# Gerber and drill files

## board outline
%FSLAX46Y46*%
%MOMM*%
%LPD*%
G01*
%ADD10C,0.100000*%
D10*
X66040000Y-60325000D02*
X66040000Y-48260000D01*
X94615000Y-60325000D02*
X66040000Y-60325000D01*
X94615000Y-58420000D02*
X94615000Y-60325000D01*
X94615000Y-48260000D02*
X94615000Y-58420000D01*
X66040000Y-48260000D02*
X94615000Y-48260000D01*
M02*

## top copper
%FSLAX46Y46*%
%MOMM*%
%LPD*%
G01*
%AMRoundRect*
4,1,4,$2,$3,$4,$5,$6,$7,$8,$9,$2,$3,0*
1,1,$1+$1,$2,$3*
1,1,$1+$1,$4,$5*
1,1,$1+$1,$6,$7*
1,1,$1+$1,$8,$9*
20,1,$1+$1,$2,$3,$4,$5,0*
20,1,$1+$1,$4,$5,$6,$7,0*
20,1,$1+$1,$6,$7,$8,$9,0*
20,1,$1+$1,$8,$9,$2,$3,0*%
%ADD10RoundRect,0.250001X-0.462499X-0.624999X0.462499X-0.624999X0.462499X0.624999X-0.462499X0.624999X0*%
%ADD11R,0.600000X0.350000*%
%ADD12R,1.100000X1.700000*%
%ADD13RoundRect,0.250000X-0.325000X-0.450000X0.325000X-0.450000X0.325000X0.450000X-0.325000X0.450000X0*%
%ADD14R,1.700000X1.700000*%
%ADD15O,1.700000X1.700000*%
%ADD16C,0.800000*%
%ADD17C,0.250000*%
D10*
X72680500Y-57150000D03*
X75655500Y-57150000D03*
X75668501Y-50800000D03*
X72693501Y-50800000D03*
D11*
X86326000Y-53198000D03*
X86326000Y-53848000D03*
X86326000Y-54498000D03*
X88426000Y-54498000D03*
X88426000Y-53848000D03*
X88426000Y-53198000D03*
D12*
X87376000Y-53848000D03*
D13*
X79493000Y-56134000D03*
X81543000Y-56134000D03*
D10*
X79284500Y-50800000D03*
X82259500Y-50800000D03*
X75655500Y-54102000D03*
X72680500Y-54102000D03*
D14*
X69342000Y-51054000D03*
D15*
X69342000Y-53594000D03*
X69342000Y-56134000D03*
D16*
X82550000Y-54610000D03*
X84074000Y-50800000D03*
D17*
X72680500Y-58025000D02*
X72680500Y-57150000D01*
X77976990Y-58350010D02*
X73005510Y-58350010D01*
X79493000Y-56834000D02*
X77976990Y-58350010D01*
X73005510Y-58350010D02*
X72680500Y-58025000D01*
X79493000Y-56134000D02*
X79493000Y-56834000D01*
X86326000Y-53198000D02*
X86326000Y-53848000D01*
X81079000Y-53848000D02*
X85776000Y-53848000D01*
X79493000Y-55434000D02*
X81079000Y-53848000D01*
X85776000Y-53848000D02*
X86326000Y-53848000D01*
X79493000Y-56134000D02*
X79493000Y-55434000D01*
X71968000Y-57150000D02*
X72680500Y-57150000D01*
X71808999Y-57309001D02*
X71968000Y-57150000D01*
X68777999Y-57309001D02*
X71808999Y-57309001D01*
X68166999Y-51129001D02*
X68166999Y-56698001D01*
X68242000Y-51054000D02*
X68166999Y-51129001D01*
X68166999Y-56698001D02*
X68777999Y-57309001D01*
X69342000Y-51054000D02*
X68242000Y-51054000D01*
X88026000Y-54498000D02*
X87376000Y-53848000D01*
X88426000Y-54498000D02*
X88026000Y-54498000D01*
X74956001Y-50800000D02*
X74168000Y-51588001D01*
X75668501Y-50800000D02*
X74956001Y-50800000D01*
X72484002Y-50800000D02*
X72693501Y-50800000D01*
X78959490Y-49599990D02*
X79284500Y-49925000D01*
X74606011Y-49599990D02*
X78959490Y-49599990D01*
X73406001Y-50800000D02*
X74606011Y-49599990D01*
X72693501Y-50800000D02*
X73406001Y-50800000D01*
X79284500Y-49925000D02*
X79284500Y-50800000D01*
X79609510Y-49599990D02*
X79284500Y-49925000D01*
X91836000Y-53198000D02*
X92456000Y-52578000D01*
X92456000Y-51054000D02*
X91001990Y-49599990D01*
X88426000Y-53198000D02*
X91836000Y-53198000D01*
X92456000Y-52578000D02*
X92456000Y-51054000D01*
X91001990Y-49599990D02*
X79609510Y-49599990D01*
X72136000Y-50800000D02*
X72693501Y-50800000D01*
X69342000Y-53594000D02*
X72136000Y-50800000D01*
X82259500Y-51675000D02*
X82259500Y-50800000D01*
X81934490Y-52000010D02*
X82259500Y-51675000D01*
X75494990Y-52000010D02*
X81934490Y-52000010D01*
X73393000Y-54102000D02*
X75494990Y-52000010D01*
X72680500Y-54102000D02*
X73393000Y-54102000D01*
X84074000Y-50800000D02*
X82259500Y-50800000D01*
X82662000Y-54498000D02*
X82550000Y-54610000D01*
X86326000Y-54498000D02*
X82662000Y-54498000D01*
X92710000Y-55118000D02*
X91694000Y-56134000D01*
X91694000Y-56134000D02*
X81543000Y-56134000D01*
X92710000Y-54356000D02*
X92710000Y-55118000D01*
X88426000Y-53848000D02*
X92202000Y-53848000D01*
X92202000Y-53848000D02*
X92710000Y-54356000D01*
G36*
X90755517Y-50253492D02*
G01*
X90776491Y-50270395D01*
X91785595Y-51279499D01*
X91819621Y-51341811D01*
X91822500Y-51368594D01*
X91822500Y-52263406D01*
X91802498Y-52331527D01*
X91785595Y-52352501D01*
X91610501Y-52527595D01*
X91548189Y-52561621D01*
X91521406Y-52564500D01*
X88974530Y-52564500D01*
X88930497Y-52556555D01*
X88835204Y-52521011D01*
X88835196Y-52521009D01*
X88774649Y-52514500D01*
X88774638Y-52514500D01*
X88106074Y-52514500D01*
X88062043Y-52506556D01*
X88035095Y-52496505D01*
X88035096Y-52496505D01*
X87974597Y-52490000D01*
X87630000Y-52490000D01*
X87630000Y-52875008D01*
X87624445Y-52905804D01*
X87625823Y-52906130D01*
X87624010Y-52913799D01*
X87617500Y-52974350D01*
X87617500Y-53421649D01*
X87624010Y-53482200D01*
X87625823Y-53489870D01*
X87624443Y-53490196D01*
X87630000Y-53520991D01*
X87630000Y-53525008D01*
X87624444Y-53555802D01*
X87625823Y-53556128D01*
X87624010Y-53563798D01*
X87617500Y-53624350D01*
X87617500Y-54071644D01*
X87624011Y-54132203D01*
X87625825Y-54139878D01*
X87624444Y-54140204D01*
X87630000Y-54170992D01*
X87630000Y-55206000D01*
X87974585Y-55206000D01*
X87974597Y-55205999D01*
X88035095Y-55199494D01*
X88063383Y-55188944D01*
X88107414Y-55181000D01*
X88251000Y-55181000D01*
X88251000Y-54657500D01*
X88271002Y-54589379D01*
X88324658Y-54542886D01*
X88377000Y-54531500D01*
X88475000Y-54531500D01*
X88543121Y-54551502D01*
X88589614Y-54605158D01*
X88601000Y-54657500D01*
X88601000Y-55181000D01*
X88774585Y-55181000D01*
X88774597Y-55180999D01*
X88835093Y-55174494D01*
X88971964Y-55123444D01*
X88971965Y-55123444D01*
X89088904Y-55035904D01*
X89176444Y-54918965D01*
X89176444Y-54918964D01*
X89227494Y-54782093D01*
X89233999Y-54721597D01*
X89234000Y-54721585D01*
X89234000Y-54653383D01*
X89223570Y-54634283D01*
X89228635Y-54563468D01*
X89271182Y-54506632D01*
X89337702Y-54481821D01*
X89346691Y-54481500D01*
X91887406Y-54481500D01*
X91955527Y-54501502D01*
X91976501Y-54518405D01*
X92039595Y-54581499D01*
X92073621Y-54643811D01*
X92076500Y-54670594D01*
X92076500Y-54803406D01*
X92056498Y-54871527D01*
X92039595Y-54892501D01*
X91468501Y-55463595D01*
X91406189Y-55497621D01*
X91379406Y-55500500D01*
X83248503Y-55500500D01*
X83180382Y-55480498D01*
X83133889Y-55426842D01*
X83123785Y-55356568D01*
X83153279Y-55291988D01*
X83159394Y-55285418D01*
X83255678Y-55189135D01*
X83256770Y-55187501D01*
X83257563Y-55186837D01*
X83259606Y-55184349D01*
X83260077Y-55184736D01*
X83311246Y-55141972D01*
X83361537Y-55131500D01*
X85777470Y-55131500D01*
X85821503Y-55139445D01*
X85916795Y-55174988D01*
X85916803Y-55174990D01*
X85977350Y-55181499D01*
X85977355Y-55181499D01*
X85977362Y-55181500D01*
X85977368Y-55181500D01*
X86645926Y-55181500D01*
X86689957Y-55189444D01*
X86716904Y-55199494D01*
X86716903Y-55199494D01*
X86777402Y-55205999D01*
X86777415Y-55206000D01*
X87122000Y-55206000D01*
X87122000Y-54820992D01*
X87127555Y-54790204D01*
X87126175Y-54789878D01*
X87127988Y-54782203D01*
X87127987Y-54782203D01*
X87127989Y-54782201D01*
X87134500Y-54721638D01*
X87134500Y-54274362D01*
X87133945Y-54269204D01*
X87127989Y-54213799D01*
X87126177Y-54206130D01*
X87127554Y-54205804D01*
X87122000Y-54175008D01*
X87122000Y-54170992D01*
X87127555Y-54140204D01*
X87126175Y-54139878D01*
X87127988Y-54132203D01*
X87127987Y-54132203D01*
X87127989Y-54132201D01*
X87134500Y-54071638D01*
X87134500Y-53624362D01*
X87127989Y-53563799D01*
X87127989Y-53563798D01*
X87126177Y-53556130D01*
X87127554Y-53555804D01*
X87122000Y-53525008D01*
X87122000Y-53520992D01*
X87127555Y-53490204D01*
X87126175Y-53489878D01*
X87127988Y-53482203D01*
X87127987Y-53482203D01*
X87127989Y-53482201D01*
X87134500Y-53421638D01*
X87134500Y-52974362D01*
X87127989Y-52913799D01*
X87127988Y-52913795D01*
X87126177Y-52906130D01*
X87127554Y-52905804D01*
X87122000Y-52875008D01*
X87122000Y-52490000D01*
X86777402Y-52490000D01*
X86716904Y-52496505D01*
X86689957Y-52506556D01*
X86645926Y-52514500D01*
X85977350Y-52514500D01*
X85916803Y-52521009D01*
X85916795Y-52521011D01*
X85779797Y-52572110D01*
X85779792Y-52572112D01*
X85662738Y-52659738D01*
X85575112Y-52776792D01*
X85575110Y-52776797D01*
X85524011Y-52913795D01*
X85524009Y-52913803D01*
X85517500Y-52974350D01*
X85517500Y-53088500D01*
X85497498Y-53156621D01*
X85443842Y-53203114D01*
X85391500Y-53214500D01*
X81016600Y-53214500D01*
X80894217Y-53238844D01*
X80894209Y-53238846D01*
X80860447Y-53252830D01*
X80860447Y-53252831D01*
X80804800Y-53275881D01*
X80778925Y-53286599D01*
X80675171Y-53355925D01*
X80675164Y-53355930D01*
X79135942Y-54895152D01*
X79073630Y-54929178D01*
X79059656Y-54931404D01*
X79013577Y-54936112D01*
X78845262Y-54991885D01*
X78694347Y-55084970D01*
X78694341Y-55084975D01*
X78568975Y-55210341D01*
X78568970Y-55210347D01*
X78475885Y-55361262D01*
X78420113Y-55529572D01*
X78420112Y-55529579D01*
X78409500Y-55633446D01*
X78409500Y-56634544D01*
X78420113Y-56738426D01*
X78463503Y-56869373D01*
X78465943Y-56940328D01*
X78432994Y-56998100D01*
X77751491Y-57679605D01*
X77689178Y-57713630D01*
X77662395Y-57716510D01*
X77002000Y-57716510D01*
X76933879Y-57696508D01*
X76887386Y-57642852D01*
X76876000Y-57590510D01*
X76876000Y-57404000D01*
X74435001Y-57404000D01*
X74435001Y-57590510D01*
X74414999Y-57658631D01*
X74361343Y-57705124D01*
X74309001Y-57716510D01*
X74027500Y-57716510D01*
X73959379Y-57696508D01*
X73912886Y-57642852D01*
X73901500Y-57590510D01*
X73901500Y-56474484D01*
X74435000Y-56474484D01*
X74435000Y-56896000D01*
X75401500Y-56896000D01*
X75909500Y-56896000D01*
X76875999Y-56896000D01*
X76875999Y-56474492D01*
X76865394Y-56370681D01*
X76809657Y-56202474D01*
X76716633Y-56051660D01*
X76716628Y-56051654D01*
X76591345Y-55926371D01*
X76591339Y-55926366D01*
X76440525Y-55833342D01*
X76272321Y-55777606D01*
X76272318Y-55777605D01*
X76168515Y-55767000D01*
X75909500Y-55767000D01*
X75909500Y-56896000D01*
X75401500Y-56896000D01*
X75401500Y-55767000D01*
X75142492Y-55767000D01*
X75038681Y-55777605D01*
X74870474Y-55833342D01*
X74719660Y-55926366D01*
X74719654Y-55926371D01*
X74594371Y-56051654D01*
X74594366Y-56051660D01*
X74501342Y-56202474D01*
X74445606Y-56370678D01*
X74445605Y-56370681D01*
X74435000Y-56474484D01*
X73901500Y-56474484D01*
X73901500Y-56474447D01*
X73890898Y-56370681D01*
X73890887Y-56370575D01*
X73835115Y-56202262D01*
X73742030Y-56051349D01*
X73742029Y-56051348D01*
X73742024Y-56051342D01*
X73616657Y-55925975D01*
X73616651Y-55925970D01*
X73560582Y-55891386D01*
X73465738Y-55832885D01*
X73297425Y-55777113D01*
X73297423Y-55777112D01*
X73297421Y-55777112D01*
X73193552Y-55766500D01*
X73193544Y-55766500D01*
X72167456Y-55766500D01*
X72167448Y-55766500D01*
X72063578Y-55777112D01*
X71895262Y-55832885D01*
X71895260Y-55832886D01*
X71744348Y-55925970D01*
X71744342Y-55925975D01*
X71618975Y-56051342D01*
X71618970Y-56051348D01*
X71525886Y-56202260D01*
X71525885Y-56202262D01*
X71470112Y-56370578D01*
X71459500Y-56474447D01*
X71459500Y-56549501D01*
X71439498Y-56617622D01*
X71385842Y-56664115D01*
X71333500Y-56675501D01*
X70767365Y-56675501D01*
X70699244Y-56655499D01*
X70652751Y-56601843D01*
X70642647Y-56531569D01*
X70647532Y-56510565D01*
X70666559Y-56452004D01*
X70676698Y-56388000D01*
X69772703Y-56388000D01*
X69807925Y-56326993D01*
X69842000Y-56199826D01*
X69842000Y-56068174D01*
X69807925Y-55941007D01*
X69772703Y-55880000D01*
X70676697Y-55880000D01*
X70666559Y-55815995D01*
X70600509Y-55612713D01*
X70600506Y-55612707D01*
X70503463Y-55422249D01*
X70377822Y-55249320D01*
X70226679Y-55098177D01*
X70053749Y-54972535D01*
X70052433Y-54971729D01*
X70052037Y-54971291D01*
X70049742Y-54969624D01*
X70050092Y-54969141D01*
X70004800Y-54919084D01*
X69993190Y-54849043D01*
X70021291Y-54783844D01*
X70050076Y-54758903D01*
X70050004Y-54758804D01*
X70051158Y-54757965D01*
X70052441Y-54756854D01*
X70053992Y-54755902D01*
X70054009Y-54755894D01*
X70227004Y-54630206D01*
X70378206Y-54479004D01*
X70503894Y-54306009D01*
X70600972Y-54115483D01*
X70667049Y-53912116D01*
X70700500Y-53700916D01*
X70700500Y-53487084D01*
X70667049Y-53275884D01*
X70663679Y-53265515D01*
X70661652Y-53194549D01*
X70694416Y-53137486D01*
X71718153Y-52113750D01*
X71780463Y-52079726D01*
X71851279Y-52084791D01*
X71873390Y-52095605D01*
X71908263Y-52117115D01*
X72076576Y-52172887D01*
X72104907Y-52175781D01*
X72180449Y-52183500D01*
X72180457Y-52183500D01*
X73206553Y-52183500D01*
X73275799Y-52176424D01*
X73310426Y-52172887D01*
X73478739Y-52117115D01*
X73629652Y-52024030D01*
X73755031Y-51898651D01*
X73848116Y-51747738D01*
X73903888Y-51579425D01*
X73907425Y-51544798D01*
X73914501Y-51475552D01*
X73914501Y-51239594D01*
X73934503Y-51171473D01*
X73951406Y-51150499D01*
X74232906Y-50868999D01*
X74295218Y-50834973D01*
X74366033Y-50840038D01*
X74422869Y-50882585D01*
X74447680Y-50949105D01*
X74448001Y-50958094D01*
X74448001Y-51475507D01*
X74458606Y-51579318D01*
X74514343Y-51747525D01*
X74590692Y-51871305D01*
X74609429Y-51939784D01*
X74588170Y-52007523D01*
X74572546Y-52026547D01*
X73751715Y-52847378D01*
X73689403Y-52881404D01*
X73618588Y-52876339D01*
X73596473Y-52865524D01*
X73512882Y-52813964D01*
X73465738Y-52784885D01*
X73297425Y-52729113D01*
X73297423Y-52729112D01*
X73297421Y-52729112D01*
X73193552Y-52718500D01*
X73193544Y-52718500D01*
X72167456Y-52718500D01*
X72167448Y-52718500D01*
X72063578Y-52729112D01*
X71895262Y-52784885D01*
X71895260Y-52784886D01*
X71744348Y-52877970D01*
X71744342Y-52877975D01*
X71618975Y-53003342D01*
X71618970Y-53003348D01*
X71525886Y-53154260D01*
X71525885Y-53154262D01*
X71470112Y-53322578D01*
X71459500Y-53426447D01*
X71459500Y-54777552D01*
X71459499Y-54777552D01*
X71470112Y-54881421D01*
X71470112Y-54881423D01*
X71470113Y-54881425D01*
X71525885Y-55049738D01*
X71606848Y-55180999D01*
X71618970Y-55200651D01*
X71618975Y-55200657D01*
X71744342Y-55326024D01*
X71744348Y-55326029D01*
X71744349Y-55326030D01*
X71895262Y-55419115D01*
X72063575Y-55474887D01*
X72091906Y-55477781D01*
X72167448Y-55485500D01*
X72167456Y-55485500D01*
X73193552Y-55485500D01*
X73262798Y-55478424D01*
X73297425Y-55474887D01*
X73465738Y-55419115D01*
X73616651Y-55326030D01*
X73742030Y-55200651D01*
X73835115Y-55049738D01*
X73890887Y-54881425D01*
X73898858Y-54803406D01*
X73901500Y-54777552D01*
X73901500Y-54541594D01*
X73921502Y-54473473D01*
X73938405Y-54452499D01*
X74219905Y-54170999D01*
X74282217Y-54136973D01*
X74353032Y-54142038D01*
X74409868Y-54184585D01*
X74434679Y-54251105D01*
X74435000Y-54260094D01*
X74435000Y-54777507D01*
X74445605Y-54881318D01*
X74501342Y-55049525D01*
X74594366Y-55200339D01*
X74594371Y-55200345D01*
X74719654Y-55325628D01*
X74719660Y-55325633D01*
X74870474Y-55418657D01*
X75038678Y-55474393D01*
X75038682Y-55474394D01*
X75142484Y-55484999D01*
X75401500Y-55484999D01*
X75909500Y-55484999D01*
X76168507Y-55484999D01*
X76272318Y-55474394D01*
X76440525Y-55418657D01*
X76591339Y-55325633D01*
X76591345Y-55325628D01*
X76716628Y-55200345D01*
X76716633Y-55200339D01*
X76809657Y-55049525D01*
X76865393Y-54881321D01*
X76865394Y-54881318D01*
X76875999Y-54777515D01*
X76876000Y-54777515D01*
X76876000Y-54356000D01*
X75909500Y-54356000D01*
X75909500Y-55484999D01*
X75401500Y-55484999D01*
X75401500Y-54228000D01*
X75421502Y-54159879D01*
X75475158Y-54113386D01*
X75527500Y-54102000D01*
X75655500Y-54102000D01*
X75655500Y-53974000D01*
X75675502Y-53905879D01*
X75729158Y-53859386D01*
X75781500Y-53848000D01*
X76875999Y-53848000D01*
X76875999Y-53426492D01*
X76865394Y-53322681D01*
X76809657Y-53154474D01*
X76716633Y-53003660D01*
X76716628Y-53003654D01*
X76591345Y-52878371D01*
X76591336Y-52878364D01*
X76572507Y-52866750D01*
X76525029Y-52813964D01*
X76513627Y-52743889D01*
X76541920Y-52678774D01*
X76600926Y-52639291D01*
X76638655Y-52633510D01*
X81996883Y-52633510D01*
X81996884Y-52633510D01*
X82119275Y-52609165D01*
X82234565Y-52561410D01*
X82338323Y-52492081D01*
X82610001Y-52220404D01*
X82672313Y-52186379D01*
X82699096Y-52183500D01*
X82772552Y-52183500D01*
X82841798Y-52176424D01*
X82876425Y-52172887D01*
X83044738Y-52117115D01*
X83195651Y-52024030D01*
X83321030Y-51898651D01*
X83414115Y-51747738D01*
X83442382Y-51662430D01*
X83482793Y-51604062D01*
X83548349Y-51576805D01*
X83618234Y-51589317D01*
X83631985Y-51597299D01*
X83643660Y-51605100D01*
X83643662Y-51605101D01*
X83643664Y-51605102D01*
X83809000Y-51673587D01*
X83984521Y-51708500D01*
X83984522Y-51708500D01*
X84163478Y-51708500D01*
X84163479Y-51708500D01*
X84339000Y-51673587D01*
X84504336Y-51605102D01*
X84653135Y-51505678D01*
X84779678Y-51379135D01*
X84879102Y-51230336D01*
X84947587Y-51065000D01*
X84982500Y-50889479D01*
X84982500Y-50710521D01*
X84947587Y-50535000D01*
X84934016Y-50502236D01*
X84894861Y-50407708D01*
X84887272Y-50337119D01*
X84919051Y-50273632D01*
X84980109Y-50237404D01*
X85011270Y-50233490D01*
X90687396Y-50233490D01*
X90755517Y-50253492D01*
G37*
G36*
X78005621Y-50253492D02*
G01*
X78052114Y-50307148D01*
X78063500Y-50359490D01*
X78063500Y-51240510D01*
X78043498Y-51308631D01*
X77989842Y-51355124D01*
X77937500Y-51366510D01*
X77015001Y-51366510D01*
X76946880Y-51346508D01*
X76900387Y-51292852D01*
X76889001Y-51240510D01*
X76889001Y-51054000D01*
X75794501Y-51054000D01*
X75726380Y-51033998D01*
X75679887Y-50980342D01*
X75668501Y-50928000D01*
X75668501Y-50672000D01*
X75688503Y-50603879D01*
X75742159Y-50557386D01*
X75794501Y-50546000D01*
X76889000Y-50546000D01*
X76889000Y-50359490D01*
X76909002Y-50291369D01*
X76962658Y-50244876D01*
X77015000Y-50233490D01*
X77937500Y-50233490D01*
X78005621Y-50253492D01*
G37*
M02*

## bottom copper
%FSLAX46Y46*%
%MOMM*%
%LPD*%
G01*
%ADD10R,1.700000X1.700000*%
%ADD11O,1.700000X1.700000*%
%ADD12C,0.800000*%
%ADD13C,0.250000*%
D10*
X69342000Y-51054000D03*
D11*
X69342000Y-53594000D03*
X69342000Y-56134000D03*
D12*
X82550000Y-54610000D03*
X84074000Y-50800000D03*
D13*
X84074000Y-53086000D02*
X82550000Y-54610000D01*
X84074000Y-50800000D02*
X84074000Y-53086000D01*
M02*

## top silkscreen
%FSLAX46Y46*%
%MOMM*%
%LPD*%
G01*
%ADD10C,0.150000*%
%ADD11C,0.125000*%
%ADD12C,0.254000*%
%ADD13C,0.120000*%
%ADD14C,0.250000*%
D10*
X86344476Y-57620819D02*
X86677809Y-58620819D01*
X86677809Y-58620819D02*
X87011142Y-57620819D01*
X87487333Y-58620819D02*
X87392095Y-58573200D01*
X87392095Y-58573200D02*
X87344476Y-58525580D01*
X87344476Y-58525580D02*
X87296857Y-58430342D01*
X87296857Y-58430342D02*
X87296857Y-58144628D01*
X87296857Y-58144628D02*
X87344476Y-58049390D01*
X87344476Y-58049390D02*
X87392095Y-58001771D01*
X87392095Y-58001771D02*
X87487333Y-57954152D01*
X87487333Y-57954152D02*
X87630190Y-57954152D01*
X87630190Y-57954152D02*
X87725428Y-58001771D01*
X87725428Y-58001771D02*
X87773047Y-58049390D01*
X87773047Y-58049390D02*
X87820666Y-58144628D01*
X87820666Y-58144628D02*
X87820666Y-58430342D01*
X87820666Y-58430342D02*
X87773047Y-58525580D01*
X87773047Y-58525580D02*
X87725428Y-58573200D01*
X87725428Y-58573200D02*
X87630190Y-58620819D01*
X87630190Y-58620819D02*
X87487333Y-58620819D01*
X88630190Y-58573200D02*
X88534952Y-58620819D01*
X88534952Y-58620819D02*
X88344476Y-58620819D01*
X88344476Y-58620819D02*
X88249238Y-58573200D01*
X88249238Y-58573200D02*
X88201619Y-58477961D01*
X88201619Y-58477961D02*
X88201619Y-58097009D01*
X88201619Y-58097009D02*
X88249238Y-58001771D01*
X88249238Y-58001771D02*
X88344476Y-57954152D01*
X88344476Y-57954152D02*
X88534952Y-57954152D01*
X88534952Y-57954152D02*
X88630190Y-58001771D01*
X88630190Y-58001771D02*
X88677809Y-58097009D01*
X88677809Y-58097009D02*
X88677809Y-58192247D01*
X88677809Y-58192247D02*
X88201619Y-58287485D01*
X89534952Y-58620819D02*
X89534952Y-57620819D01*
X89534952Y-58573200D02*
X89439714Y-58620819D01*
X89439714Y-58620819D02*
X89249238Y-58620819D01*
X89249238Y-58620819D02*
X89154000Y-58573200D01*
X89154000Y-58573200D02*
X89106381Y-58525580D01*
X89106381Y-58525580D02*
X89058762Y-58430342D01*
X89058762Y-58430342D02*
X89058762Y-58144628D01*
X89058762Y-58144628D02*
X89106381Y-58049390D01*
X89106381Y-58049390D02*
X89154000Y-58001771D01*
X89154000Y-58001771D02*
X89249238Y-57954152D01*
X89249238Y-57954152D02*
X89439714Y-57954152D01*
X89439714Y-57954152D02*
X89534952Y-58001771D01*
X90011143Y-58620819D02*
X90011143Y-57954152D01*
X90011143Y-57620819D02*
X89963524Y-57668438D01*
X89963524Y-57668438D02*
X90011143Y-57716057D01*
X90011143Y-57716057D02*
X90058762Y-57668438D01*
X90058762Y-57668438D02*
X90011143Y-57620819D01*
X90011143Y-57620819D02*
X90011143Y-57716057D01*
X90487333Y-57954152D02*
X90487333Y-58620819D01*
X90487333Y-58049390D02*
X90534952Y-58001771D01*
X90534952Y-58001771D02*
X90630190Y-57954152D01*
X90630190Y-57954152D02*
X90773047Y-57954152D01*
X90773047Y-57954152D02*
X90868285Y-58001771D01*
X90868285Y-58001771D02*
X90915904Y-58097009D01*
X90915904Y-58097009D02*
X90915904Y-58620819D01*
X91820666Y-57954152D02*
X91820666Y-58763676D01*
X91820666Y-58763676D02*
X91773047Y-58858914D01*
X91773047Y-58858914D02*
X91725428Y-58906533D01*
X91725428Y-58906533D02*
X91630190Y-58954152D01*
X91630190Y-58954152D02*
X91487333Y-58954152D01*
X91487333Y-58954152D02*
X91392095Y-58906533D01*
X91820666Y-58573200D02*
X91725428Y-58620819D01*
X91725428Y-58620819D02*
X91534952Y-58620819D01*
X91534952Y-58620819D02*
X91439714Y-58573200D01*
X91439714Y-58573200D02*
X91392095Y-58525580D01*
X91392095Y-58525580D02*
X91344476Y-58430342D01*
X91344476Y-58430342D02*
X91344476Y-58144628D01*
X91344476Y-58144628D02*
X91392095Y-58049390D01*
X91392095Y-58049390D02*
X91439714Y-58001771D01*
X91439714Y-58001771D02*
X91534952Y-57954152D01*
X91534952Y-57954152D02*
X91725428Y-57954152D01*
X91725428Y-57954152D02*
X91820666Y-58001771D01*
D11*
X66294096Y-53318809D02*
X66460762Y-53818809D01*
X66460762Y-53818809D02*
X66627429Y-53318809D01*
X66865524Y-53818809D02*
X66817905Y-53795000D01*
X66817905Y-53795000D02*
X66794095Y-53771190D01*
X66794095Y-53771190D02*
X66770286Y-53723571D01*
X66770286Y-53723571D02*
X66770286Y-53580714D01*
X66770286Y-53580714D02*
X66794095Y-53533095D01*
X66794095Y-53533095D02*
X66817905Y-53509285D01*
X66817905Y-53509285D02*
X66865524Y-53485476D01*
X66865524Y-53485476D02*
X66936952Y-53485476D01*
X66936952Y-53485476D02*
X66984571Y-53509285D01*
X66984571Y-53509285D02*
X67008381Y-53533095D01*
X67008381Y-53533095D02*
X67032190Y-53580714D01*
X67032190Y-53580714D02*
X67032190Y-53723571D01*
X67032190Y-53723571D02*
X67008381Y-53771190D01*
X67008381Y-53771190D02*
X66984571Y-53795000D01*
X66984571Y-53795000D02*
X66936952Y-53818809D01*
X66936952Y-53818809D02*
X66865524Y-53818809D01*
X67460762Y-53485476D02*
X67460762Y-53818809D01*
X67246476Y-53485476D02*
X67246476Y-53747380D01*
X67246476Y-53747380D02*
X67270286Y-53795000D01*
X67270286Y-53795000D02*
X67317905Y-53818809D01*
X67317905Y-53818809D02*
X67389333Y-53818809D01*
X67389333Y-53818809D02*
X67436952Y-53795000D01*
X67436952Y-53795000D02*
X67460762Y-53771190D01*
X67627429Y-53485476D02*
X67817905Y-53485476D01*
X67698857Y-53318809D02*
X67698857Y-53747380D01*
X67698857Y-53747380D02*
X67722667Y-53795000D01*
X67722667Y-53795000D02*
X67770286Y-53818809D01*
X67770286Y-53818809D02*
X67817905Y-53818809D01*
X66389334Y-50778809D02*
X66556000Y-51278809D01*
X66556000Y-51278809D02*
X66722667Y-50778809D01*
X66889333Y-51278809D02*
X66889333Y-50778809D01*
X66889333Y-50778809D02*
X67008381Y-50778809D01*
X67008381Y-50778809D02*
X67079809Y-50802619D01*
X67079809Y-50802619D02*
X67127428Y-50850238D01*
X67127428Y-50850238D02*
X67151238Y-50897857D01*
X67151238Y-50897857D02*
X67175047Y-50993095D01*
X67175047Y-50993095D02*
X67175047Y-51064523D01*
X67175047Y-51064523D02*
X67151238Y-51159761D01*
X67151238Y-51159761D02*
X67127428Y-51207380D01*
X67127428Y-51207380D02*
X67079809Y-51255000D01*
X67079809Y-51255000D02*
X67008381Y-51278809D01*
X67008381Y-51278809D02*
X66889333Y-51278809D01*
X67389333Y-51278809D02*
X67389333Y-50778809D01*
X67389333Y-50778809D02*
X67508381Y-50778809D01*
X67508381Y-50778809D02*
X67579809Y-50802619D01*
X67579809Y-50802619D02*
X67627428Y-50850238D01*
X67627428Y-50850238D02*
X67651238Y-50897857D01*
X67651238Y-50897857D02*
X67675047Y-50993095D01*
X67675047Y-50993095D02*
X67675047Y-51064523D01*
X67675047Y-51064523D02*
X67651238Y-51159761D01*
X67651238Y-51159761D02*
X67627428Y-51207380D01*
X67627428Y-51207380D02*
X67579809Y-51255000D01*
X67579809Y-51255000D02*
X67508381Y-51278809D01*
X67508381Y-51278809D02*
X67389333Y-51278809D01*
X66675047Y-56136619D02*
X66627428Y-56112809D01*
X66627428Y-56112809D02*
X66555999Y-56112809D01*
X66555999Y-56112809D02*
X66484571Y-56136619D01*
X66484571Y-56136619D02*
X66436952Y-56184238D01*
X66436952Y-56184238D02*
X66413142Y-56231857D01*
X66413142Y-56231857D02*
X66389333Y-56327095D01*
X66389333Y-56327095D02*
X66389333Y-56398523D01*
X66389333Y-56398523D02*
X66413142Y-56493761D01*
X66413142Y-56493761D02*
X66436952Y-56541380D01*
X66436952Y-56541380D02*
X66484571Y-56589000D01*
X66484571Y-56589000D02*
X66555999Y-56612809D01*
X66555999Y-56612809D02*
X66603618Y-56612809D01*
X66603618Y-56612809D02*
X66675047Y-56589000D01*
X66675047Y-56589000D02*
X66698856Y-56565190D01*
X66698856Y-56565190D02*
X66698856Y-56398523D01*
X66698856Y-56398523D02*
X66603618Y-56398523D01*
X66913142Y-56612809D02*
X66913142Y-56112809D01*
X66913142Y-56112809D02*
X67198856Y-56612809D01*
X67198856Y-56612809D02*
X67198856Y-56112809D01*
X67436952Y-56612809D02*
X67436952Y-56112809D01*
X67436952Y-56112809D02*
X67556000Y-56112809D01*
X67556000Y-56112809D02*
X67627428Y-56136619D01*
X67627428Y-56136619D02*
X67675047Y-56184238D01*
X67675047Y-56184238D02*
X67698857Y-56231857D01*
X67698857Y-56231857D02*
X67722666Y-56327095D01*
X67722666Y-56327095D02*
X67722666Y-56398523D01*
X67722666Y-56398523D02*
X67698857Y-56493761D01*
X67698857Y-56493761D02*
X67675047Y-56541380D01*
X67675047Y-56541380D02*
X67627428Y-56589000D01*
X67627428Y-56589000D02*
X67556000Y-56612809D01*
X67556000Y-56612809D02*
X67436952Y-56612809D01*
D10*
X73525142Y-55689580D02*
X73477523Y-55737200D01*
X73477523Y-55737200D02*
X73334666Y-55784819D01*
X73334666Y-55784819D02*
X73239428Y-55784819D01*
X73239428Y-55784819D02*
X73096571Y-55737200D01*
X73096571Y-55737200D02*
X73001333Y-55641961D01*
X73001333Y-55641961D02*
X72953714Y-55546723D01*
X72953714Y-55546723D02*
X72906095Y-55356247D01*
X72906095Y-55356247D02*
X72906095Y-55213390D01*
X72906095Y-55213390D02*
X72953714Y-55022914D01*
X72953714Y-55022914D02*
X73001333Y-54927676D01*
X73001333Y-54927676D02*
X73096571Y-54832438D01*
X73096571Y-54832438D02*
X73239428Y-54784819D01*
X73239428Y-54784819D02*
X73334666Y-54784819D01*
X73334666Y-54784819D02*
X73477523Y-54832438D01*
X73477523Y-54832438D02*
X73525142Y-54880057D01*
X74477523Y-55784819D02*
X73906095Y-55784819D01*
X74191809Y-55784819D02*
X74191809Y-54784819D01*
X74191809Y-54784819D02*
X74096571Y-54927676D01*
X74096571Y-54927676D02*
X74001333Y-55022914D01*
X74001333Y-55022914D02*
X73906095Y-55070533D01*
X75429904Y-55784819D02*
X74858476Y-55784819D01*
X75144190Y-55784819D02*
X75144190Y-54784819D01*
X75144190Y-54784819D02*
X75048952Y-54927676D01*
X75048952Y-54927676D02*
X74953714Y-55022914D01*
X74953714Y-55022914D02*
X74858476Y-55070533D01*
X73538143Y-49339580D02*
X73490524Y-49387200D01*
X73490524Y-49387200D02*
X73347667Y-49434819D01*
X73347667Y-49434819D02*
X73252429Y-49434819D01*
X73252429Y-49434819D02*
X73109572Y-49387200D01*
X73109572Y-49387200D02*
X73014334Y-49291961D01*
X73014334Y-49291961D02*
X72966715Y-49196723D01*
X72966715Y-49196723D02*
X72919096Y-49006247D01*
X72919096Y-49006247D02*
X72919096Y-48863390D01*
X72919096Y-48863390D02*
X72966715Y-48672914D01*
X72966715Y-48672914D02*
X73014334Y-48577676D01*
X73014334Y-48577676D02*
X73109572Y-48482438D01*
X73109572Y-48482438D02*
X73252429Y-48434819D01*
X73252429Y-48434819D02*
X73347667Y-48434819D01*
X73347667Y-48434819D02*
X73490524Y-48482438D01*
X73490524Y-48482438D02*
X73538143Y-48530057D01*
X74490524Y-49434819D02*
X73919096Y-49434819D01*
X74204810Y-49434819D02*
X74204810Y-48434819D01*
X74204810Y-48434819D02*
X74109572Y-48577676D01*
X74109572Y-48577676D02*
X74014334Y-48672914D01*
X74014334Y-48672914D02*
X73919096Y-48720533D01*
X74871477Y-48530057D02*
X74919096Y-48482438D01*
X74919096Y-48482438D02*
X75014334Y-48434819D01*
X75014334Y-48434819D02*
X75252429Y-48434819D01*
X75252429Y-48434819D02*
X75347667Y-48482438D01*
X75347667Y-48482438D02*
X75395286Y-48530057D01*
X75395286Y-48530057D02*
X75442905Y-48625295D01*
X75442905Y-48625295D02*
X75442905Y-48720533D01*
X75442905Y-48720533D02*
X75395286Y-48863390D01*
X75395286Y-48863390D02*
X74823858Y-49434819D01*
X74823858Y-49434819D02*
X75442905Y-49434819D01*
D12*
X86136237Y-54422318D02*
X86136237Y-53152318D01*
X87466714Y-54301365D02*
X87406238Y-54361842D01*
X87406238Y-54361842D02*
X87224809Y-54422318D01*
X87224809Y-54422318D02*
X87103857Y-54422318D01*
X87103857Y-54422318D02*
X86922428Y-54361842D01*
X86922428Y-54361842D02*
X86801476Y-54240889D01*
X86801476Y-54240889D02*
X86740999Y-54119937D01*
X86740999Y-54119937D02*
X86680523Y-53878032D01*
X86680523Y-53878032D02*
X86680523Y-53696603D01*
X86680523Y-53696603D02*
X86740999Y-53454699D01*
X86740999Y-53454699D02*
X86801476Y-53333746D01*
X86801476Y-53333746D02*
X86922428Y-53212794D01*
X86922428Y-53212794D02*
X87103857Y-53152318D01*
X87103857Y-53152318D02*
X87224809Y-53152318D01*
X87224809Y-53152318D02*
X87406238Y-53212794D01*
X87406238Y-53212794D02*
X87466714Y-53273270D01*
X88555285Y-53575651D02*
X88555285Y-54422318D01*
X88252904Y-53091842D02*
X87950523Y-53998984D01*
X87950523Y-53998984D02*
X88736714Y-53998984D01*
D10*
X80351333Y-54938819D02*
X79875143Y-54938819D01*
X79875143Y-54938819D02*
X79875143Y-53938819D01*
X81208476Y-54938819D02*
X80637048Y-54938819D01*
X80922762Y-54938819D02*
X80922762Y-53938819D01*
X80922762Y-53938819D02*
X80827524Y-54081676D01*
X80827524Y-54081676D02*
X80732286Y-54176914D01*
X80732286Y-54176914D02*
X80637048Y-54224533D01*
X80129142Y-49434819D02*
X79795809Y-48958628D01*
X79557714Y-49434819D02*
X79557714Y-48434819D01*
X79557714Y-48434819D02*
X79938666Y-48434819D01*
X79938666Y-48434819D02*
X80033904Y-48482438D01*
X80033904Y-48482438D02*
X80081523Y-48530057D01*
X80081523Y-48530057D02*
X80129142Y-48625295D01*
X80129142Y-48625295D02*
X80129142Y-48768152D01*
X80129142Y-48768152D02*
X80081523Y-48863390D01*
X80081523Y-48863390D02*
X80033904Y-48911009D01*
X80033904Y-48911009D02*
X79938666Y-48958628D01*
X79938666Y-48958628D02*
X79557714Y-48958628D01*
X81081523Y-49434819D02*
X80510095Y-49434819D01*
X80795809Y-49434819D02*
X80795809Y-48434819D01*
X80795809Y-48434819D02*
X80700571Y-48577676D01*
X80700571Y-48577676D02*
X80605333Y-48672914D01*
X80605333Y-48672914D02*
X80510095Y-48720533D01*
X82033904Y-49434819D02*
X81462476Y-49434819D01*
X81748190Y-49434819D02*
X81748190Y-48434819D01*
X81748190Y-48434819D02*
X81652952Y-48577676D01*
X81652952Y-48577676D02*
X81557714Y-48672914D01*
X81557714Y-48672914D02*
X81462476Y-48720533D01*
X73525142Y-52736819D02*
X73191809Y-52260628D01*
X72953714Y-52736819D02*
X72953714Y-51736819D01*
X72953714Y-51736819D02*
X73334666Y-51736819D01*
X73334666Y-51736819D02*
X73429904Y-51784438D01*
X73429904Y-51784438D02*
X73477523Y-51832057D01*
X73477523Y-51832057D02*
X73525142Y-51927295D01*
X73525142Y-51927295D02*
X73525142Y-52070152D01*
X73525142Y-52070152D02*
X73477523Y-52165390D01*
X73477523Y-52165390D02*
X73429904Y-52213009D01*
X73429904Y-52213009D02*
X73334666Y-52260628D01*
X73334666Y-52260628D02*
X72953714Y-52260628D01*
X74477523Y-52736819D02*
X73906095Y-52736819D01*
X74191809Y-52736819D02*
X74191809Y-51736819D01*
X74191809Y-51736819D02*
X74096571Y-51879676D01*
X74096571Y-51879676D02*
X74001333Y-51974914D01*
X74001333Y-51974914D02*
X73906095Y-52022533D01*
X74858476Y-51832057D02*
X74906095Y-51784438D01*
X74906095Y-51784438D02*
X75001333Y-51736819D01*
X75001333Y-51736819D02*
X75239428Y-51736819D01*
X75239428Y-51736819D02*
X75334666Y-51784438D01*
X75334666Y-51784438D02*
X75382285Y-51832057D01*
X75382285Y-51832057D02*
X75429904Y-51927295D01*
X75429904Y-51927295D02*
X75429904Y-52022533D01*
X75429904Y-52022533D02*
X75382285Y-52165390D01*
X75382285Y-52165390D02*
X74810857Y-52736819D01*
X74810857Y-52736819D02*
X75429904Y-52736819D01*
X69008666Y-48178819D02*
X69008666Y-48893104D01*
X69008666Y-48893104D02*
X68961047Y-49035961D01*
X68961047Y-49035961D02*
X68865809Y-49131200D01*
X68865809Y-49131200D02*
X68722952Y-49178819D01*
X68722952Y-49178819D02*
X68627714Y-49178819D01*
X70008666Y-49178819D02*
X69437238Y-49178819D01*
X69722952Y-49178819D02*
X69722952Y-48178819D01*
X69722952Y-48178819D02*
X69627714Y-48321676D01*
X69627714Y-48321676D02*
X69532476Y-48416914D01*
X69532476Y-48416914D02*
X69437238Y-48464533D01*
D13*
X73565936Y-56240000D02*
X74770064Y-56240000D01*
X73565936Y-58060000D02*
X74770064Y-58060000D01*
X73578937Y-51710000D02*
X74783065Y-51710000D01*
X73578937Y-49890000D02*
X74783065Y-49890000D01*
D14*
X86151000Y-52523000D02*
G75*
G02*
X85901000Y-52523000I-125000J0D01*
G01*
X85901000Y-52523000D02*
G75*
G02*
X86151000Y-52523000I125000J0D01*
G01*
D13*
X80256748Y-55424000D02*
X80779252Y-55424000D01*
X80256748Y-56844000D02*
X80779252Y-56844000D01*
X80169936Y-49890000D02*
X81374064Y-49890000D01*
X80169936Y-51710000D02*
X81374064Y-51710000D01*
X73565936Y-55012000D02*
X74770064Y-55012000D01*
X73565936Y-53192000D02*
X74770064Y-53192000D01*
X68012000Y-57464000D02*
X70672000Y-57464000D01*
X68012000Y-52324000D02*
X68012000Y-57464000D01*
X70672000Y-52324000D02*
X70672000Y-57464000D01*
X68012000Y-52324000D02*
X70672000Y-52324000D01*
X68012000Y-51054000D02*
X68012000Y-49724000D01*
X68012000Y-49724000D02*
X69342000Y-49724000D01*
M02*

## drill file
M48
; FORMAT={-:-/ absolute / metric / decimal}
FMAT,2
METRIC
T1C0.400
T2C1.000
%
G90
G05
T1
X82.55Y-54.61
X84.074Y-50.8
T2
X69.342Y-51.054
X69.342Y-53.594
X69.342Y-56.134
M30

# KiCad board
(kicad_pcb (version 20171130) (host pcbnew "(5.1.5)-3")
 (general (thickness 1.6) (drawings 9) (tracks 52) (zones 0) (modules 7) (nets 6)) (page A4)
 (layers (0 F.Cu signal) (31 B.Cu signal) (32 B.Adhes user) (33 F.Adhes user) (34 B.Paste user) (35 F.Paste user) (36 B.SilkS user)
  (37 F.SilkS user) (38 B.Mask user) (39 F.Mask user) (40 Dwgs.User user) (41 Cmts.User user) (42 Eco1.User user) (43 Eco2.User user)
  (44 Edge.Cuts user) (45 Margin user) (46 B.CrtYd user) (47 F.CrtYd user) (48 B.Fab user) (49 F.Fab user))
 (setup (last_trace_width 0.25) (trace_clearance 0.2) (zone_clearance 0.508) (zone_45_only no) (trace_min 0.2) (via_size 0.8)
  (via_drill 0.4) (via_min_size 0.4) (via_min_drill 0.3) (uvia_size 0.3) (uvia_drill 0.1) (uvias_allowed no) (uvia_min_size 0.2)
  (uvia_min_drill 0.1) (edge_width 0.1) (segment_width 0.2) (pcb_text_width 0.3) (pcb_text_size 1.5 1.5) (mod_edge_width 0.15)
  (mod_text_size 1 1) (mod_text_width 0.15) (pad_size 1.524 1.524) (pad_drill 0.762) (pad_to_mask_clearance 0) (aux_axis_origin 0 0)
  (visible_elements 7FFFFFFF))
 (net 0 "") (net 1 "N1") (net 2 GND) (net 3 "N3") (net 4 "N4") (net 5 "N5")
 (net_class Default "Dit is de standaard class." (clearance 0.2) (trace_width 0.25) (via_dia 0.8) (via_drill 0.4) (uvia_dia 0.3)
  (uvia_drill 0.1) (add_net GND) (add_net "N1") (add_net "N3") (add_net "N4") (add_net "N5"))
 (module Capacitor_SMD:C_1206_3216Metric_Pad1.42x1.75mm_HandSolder (layer F.Cu) (at 74.168 57.15)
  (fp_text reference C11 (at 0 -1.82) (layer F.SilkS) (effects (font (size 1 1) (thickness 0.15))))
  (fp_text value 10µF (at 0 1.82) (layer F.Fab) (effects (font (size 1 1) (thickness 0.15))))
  (fp_line (start -0.602064 -0.91) (end 0.602064 -0.91) (layer F.SilkS) (width 0.12))
  (fp_line (start -0.602064 0.91) (end 0.602064 0.91) (layer F.SilkS) (width 0.12))
  (pad 1 smd roundrect (at -1.4875 0) (size 1.425 1.75) (layers F.Cu F.Paste F.Mask) (roundrect_rratio 0.175439) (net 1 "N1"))
  (pad 2 smd roundrect (at 1.4875 0) (size 1.425 1.75) (layers F.Cu F.Paste F.Mask) (roundrect_rratio 0.175439) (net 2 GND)))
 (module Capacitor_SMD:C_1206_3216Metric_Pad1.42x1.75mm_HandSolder (layer F.Cu) (at 74.181001 50.8)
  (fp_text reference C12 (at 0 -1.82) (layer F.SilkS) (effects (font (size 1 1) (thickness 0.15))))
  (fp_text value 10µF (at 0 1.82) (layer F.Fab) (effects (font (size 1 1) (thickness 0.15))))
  (fp_line (start -0.602064 0.91) (end 0.602064 0.91) (layer F.SilkS) (width 0.12))
  (fp_line (start -0.602064 -0.91) (end 0.602064 -0.91) (layer F.SilkS) (width 0.12))
  (pad 2 smd roundrect (at 1.4875 0) (size 1.425 1.75) (layers F.Cu F.Paste F.Mask) (roundrect_rratio 0.175439) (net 2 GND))
  (pad 1 smd roundrect (at -1.4875 0) (size 1.425 1.75) (layers F.Cu F.Paste F.Mask) (roundrect_rratio 0.175439) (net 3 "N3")))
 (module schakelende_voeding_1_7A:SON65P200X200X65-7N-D (layer F.Cu) (at 87.376 53.848)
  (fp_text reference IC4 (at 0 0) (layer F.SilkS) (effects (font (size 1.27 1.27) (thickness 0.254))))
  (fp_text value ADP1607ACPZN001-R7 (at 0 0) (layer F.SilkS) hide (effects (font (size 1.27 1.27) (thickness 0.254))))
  (fp_circle (center -1.35 -1.325) (end -1.35 -1.2) (layer F.SilkS) (width 0.25))
  (pad 1 smd rect (at -1.05 -0.65 90) (size 0.35 0.6) (layers F.Cu F.Paste F.Mask) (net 1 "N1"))
  (pad 2 smd rect (at -1.05 0 90) (size 0.35 0.6) (layers F.Cu F.Paste F.Mask) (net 1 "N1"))
  (pad 3 smd rect (at -1.05 0.65 90) (size 0.35 0.6) (layers F.Cu F.Paste F.Mask) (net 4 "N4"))
  (pad 4 smd rect (at 1.05 0.65 90) (size 0.35 0.6) (layers F.Cu F.Paste F.Mask) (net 2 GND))
  (pad 5 smd rect (at 1.05 0 90) (size 0.35 0.6) (layers F.Cu F.Paste F.Mask) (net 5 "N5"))
  (pad 6 smd rect (at 1.05 -0.65 90) (size 0.35 0.6) (layers F.Cu F.Paste F.Mask) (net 3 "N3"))
  (pad 7 smd rect (at 0 0) (size 1.1 1.7) (layers F.Cu F.Paste F.Mask) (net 2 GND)))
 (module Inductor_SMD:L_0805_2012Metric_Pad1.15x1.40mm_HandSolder (layer F.Cu) (at 80.518 56.134)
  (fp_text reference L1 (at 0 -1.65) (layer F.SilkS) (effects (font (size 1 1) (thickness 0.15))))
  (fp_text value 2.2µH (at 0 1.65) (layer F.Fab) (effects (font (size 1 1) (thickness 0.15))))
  (fp_line (start -0.261252 -0.71) (end 0.261252 -0.71) (layer F.SilkS) (width 0.12))
  (fp_line (start -0.261252 0.71) (end 0.261252 0.71) (layer F.SilkS) (width 0.12))
  (pad 1 smd roundrect (at -1.025 0) (size 1.15 1.4) (layers F.Cu F.Paste F.Mask) (roundrect_rratio 0.217391) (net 1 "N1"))
  (pad 2 smd roundrect (at 1.025 0) (size 1.15 1.4) (layers F.Cu F.Paste F.Mask) (roundrect_rratio 0.217391) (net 5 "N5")))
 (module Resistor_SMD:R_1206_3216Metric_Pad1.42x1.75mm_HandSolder (layer F.Cu) (at 80.772 50.8)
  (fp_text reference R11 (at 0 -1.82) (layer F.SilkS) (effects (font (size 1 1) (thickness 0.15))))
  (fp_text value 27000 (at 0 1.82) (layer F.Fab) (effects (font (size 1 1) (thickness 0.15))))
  (fp_line (start -0.602064 -0.91) (end 0.602064 -0.91) (layer F.SilkS) (width 0.12))
  (fp_line (start -0.602064 0.91) (end 0.602064 0.91) (layer F.SilkS) (width 0.12))
  (pad 1 smd roundrect (at -1.4875 0) (size 1.425 1.75) (layers F.Cu F.Paste F.Mask) (roundrect_rratio 0.175439) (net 3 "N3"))
  (pad 2 smd roundrect (at 1.4875 0) (size 1.425 1.75) (layers F.Cu F.Paste F.Mask) (roundrect_rratio 0.175439) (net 4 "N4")))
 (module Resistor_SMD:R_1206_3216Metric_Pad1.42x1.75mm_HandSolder (layer F.Cu) (at 74.168 54.102)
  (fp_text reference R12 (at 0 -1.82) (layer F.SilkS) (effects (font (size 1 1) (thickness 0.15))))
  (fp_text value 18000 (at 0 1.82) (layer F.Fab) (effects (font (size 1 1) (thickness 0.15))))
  (fp_line (start -0.602064 0.91) (end 0.602064 0.91) (layer F.SilkS) (width 0.12))
  (fp_line (start -0.602064 -0.91) (end 0.602064 -0.91) (layer F.SilkS) (width 0.12))
  (pad 2 smd roundrect (at 1.4875 0) (size 1.425 1.75) (layers F.Cu F.Paste F.Mask) (roundrect_rratio 0.175439) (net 2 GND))
  (pad 1 smd roundrect (at -1.4875 0) (size 1.425 1.75) (layers F.Cu F.Paste F.Mask) (roundrect_rratio 0.175439) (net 4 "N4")))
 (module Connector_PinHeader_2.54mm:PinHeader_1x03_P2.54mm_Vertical (layer F.Cu) (at 69.342 51.054)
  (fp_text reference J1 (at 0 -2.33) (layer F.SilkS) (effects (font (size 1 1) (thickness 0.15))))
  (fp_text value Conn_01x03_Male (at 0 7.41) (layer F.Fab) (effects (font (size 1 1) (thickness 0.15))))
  (fp_line (start -1.33 6.41) (end 1.33 6.41) (layer F.SilkS) (width 0.12))
  (fp_line (start -1.33 1.27) (end -1.33 6.41) (layer F.SilkS) (width 0.12))
  (fp_line (start 1.33 1.27) (end 1.33 6.41) (layer F.SilkS) (width 0.12))
  (fp_line (start -1.33 1.27) (end 1.33 1.27) (layer F.SilkS) (width 0.12))
  (fp_line (start -1.33 0) (end -1.33 -1.33) (layer F.SilkS) (width 0.12))
  (fp_line (start -1.33 -1.33) (end 0 -1.33) (layer F.SilkS) (width 0.12))
  (pad 1 thru_hole rect (at 0 0) (size 1.7 1.7) (drill 1) (layers *.Cu *.Mask) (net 1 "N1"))
  (pad 2 thru_hole oval (at 0 2.54) (size 1.7 1.7) (drill 1) (layers *.Cu *.Mask) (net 3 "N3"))
  (pad 3 thru_hole oval (at 0 5.08) (size 1.7 1.7) (drill 1) (layers *.Cu *.Mask) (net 2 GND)))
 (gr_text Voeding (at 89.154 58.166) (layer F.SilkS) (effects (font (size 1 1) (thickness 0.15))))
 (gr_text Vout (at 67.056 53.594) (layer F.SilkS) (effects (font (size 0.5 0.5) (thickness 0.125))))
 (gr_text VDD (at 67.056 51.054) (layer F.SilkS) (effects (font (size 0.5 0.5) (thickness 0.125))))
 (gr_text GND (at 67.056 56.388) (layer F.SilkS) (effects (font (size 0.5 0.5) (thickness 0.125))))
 (gr_line (start 66.04 60.325) (end 66.04 48.26) (layer Edge.Cuts) (width 0.1))
 (gr_line (start 94.615 60.325) (end 66.04 60.325) (layer Edge.Cuts) (width 0.1))
 (gr_line (start 94.615 58.42) (end 94.615 60.325) (layer Edge.Cuts) (width 0.1))
 (gr_line (start 94.615 48.26) (end 94.615 58.42) (layer Edge.Cuts) (width 0.1))
 (gr_line (start 66.04 48.26) (end 94.615 48.26) (layer Edge.Cuts) (width 0.1))
 (segment (start 72.6805 58.025) (end 72.6805 57.15) (width 0.25) (layer F.Cu) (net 1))
 (segment (start 77.97699 58.35001) (end 73.00551 58.35001) (width 0.25) (layer F.Cu) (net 1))
 (segment (start 79.493 56.834) (end 77.97699 58.35001) (width 0.25) (layer F.Cu) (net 1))
 (segment (start 73.00551 58.35001) (end 72.6805 58.025) (width 0.25) (layer F.Cu) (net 1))
 (segment (start 79.493 56.134) (end 79.493 56.834) (width 0.25) (layer F.Cu) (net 1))
 (segment (start 86.326 53.198) (end 86.326 53.848) (width 0.25) (layer F.Cu) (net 1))
 (segment (start 81.079 53.848) (end 85.776 53.848) (width 0.25) (layer F.Cu) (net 1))
 (segment (start 79.493 55.434) (end 81.079 53.848) (width 0.25) (layer F.Cu) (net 1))
 (segment (start 85.776 53.848) (end 86.326 53.848) (width 0.25) (layer F.Cu) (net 1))
 (segment (start 79.493 56.134) (end 79.493 55.434) (width 0.25) (layer F.Cu) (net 1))
 (segment (start 71.968 57.15) (end 72.6805 57.15) (width 0.25) (layer F.Cu) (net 1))
 (segment (start 71.808999 57.309001) (end 71.968 57.15) (width 0.25) (layer F.Cu) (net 1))
 (segment (start 68.777999 57.309001) (end 71.808999 57.309001) (width 0.25) (layer F.Cu) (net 1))
 (segment (start 68.166999 51.129001) (end 68.166999 56.698001) (width 0.25) (layer F.Cu) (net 1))
 (segment (start 68.242 51.054) (end 68.166999 51.129001) (width 0.25) (layer F.Cu) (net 1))
 (segment (start 68.166999 56.698001) (end 68.777999 57.309001) (width 0.25) (layer F.Cu) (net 1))
 (segment (start 69.342 51.054) (end 68.242 51.054) (width 0.25) (layer F.Cu) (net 1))
 (segment (start 88.026 54.498) (end 87.376 53.848) (width 0.25) (layer F.Cu) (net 2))
 (segment (start 88.426 54.498) (end 88.026 54.498) (width 0.25) (layer F.Cu) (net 2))
 (segment (start 74.956001 50.8) (end 74.168 51.588001) (width 0.25) (layer F.Cu) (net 2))
 (segment (start 75.668501 50.8) (end 74.956001 50.8) (width 0.25) (layer F.Cu) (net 2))
 (segment (start 72.484002 50.8) (end 72.693501 50.8) (width 0.25) (layer F.Cu) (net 3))
 (segment (start 78.95949 49.59999) (end 79.2845 49.925) (width 0.25) (layer F.Cu) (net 3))
 (segment (start 74.606011 49.59999) (end 78.95949 49.59999) (width 0.25) (layer F.Cu) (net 3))
 (segment (start 73.406001 50.8) (end 74.606011 49.59999) (width 0.25) (layer F.Cu) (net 3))
 (segment (start 72.693501 50.8) (end 73.406001 50.8) (width 0.25) (layer F.Cu) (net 3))
 (segment (start 79.2845 49.925) (end 79.2845 50.8) (width 0.25) (layer F.Cu) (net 3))
 (segment (start 79.60951 49.59999) (end 79.2845 49.925) (width 0.25) (layer F.Cu) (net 3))
 (segment (start 91.836 53.198) (end 92.456 52.578) (width 0.25) (layer F.Cu) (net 3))
 (segment (start 92.456 51.054) (end 91.00199 49.59999) (width 0.25) (layer F.Cu) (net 3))
 (segment (start 88.426 53.198) (end 91.836 53.198) (width 0.25) (layer F.Cu) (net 3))
 (segment (start 92.456 52.578) (end 92.456 51.054) (width 0.25) (layer F.Cu) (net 3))
 (segment (start 91.00199 49.59999) (end 79.60951 49.59999) (width 0.25) (layer F.Cu) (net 3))
 (segment (start 72.136 50.8) (end 72.693501 50.8) (width 0.25) (layer F.Cu) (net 3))
 (segment (start 69.342 53.594) (end 72.136 50.8) (width 0.25) (layer F.Cu) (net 3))
 (via (at 82.55 54.61) (size 0.8) (drill 0.4) (layers F.Cu B.Cu) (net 4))
 (via (at 84.074 50.8) (size 0.8) (drill 0.4) (layers F.Cu B.Cu) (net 4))
 (segment (start 82.2595 51.675) (end 82.2595 50.8) (width 0.25) (layer F.Cu) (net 4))
 (segment (start 81.93449 52.00001) (end 82.2595 51.675) (width 0.25) (layer F.Cu) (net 4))
 (segment (start 75.49499 52.00001) (end 81.93449 52.00001) (width 0.25) (layer F.Cu) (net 4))
 (segment (start 73.393 54.102) (end 75.49499 52.00001) (width 0.25) (layer F.Cu) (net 4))
 (segment (start 72.6805 54.102) (end 73.393 54.102) (width 0.25) (layer F.Cu) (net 4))
 (segment (start 84.074 53.086) (end 82.55 54.61) (width 0.25) (layer B.Cu) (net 4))
 (segment (start 84.074 50.8) (end 84.074 53.086) (width 0.25) (layer B.Cu) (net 4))
 (segment (start 84.074 50.8) (end 82.2595 50.8) (width 0.25) (layer F.Cu) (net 4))
 (segment (start 82.662 54.498) (end 82.55 54.61) (width 0.25) (layer F.Cu) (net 4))
 (segment (start 86.326 54.498) (end 82.662 54.498) (width 0.25) (layer F.Cu) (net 4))
 (segment (start 92.71 55.118) (end 91.694 56.134) (width 0.25) (layer F.Cu) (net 5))
 (segment (start 91.694 56.134) (end 81.543 56.134) (width 0.25) (layer F.Cu) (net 5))
 (segment (start 92.71 54.356) (end 92.71 55.118) (width 0.25) (layer F.Cu) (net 5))
 (segment (start 88.426 53.848) (end 92.202 53.848) (width 0.25) (layer F.Cu) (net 5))
 (segment (start 92.202 53.848) (end 92.71 54.356) (width 0.25) (layer F.Cu) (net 5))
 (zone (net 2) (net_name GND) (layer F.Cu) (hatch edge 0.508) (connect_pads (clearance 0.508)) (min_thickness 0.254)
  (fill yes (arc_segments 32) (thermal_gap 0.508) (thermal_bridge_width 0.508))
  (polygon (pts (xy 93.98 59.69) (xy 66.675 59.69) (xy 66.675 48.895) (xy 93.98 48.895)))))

